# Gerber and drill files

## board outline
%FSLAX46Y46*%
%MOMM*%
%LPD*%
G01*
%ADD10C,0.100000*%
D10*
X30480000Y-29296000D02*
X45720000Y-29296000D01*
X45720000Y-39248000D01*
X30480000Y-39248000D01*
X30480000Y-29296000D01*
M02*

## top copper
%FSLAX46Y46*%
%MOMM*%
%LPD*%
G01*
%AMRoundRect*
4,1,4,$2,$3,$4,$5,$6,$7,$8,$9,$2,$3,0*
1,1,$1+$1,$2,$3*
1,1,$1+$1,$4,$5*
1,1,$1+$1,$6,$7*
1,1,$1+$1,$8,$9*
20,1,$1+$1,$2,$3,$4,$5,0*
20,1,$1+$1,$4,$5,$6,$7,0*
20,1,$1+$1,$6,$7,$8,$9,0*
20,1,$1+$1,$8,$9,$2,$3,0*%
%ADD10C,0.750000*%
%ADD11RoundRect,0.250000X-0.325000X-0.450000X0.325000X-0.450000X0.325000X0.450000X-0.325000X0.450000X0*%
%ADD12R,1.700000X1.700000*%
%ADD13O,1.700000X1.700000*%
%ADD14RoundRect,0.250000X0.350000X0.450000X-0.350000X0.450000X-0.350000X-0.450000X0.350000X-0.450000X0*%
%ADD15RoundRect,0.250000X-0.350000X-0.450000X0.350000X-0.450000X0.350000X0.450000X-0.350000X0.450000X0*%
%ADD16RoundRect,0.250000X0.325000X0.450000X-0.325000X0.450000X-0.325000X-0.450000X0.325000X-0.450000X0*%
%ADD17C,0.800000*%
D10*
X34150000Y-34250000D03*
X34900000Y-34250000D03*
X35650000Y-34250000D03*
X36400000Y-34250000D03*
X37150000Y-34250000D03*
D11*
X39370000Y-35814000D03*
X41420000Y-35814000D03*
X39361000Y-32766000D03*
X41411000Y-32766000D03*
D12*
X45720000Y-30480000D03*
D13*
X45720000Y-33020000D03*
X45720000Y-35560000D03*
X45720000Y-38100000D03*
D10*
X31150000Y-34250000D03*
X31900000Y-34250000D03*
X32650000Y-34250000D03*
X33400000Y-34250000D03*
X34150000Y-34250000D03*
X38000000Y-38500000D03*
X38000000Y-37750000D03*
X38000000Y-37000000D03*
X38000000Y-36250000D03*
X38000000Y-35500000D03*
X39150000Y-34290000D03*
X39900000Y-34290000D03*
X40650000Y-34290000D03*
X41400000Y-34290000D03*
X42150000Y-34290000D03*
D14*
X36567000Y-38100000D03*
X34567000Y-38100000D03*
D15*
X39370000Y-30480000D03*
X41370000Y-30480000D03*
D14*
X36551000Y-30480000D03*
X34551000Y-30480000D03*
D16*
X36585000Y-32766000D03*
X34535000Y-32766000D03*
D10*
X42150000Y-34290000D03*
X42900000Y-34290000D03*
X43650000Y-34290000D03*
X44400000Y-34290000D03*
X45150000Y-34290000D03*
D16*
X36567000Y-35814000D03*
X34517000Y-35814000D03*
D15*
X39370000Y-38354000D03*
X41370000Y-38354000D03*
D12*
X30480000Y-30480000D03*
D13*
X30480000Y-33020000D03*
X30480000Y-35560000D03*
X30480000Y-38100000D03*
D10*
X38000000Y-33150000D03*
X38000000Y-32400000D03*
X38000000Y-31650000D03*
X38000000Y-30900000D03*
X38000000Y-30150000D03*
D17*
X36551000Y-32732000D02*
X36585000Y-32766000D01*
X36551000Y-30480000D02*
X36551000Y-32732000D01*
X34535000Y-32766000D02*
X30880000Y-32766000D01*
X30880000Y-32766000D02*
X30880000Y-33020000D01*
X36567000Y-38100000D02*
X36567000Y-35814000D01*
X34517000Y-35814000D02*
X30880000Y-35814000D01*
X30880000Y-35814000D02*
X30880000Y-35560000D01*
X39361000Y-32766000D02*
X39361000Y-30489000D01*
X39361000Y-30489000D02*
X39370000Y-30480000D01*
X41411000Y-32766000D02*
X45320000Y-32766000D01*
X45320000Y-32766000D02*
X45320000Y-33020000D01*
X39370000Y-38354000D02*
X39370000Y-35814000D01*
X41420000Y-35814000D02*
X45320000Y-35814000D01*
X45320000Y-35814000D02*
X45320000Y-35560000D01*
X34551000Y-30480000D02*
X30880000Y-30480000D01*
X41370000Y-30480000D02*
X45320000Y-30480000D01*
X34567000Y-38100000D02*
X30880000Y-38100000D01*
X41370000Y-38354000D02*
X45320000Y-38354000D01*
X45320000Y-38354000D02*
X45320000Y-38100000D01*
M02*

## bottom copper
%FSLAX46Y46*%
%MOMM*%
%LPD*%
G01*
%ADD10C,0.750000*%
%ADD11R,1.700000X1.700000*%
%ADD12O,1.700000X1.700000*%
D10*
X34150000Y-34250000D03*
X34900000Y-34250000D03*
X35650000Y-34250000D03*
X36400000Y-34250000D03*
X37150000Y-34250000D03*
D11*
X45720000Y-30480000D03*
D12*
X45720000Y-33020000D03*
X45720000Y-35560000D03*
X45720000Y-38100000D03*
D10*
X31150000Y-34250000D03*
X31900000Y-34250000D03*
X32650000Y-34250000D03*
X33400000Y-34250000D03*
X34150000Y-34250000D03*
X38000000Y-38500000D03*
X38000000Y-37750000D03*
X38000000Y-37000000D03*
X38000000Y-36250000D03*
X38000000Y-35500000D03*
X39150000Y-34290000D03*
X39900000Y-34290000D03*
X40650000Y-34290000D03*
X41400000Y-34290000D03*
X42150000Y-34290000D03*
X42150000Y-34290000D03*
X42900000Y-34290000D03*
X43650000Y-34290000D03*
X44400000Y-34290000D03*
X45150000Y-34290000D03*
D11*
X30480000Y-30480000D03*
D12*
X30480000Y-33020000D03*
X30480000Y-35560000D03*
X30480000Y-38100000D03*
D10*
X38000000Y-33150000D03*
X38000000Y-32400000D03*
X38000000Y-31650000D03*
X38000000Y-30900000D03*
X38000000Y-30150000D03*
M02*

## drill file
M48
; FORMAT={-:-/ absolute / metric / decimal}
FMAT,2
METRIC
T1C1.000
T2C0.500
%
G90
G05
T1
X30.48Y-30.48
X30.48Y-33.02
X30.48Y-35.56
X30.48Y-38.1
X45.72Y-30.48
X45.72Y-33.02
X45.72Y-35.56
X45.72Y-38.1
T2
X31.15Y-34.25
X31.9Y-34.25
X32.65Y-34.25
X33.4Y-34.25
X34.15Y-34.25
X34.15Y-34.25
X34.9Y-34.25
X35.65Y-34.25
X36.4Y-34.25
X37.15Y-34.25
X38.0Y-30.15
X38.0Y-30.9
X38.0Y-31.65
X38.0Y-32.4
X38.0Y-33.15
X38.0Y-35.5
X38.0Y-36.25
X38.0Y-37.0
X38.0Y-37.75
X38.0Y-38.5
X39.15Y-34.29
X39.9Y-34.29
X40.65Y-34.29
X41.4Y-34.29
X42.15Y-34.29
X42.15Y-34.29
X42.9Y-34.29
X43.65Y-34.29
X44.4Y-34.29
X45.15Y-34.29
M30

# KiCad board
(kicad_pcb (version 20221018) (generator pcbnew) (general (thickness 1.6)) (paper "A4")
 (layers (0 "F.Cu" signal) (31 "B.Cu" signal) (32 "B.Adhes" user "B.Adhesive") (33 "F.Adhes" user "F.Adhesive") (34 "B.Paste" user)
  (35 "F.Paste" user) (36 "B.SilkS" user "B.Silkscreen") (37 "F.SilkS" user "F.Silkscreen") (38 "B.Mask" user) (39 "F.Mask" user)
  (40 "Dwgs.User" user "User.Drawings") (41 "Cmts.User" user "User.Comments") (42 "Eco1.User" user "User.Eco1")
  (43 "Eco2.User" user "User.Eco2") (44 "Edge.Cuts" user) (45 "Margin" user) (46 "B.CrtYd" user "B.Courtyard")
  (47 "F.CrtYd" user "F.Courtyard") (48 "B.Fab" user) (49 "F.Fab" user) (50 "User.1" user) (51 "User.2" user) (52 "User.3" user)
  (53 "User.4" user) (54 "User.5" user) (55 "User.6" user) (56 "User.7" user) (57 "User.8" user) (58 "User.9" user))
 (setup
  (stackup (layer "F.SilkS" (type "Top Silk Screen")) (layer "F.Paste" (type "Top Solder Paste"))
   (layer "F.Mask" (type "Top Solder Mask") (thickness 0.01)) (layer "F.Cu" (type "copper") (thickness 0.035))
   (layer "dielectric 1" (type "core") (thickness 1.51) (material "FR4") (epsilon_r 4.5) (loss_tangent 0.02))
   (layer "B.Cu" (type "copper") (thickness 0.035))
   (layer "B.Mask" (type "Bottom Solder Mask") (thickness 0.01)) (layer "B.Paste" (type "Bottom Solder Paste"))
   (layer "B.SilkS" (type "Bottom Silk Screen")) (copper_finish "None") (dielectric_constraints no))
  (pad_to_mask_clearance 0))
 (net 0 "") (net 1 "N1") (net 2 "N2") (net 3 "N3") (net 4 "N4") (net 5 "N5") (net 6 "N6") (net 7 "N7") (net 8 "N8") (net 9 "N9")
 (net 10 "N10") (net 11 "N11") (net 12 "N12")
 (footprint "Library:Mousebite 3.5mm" (layer "F.Cu") (at 34.15 34.25 90)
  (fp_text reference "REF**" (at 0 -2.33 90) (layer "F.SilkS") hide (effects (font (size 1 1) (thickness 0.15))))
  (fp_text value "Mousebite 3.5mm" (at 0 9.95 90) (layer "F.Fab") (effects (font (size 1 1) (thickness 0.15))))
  (pad "" np_thru_hole circle (at 0 0 90) (size 0.75 0.75) (drill 0.5) (layers "*.Cu" "*.Mask"))
  (pad "" np_thru_hole circle (at 0 0.75 90) (size 0.75 0.75) (drill 0.5) (layers "*.Cu" "*.Mask"))
  (pad "" np_thru_hole circle (at 0 1.5 90) (size 0.75 0.75) (drill 0.5) (layers "*.Cu" "*.Mask"))
  (pad "" np_thru_hole circle (at 0 2.25 90) (size 0.75 0.75) (drill 0.5) (layers "*.Cu" "*.Mask"))
  (pad "" np_thru_hole circle (at 0 3 90) (size 0.75 0.75) (drill 0.5) (layers "*.Cu" "*.Mask")))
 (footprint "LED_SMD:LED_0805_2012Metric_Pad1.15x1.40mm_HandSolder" (layer "F.Cu") (at 40.395 35.814)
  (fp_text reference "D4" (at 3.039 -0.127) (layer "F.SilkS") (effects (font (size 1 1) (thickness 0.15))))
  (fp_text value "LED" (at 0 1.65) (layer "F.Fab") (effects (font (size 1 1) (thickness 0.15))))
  (pad "1" smd roundrect (at -1.025 0) (size 1.15 1.4) (layers "F.Cu" "F.Paste" "F.Mask") (roundrect_rratio 0.217391) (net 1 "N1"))
  (pad "2" smd roundrect (at 1.025 0) (size 1.15 1.4) (layers "F.Cu" "F.Paste" "F.Mask") (roundrect_rratio 0.217391) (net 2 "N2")))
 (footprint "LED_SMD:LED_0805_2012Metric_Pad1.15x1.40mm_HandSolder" (layer "F.Cu") (at 40.386 32.766)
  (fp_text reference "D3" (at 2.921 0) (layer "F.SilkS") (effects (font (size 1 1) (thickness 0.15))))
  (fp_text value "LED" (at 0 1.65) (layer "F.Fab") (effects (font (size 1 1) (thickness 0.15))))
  (pad "1" smd roundrect (at -1.025 0) (size 1.15 1.4) (layers "F.Cu" "F.Paste" "F.Mask") (roundrect_rratio 0.217391) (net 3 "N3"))
  (pad "2" smd roundrect (at 1.025 0) (size 1.15 1.4) (layers "F.Cu" "F.Paste" "F.Mask") (roundrect_rratio 0.217391) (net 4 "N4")))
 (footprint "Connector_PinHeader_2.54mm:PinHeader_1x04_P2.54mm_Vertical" (layer "F.Cu") (at 45.72 30.48)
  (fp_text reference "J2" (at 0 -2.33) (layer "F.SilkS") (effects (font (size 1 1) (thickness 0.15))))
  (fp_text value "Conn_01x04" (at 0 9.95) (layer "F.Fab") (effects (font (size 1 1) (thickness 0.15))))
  (pad "1" thru_hole rect (at 0 0) (size 1.7 1.7) (drill 1) (layers "*.Cu" "*.Mask") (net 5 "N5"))
  (pad "2" thru_hole oval (at 0 2.54) (size 1.7 1.7) (drill 1) (layers "*.Cu" "*.Mask") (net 4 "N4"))
  (pad "3" thru_hole oval (at 0 5.08) (size 1.7 1.7) (drill 1) (layers "*.Cu" "*.Mask") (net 2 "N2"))
  (pad "4" thru_hole oval (at 0 7.62) (size 1.7 1.7) (drill 1) (layers "*.Cu" "*.Mask") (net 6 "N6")))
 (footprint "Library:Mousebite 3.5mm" (layer "F.Cu") (at 31.15 34.25 90)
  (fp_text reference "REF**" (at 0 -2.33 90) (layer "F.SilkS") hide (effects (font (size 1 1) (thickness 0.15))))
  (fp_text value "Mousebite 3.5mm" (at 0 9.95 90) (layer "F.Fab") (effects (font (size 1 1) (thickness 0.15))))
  (pad "" np_thru_hole circle (at 0 0 90) (size 0.75 0.75) (drill 0.5) (layers "*.Cu" "*.Mask"))
  (pad "" np_thru_hole circle (at 0 0.75 90) (size 0.75 0.75) (drill 0.5) (layers "*.Cu" "*.Mask"))
  (pad "" np_thru_hole circle (at 0 1.5 90) (size 0.75 0.75) (drill 0.5) (layers "*.Cu" "*.Mask"))
  (pad "" np_thru_hole circle (at 0 2.25 90) (size 0.75 0.75) (drill 0.5) (layers "*.Cu" "*.Mask"))
  (pad "" np_thru_hole circle (at 0 3 90) (size 0.75 0.75) (drill 0.5) (layers "*.Cu" "*.Mask")))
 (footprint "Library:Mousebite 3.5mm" (layer "F.Cu") (at 38 38.5 180)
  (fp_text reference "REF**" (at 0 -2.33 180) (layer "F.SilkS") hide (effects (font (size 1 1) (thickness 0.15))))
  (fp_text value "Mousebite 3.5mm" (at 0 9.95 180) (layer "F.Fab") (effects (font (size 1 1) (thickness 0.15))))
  (pad "" np_thru_hole circle (at 0 0 180) (size 0.75 0.75) (drill 0.5) (layers "*.Cu" "*.Mask"))
  (pad "" np_thru_hole circle (at 0 0.75 180) (size 0.75 0.75) (drill 0.5) (layers "*.Cu" "*.Mask"))
  (pad "" np_thru_hole circle (at 0 1.5 180) (size 0.75 0.75) (drill 0.5) (layers "*.Cu" "*.Mask"))
  (pad "" np_thru_hole circle (at 0 2.25 180) (size 0.75 0.75) (drill 0.5) (layers "*.Cu" "*.Mask"))
  (pad "" np_thru_hole circle (at 0 3 180) (size 0.75 0.75) (drill 0.5) (layers "*.Cu" "*.Mask")))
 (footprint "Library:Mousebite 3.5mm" (layer "F.Cu") (at 39.15 34.29 90)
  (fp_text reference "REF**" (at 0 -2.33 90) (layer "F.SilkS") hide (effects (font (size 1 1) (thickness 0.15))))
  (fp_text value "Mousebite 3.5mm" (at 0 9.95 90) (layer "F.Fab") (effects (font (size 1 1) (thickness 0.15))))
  (pad "" np_thru_hole circle (at 0 0 90) (size 0.75 0.75) (drill 0.5) (layers "*.Cu" "*.Mask"))
  (pad "" np_thru_hole circle (at 0 0.75 90) (size 0.75 0.75) (drill 0.5) (layers "*.Cu" "*.Mask"))
  (pad "" np_thru_hole circle (at 0 1.5 90) (size 0.75 0.75) (drill 0.5) (layers "*.Cu" "*.Mask"))
  (pad "" np_thru_hole circle (at 0 2.25 90) (size 0.75 0.75) (drill 0.5) (layers "*.Cu" "*.Mask"))
  (pad "" np_thru_hole circle (at 0 3 90) (size 0.75 0.75) (drill 0.5) (layers "*.Cu" "*.Mask")))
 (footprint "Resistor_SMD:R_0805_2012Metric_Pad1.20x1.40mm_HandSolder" (layer "F.Cu") (at 35.567 38.1 180)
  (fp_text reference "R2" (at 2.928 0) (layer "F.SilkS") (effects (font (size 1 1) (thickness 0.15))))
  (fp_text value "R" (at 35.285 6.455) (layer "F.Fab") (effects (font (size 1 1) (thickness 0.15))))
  (pad "1" smd roundrect (at -1 0 180) (size 1.2 1.4) (layers "F.Cu" "F.Paste" "F.Mask") (roundrect_rratio 0.208333) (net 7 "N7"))
  (pad "2" smd roundrect (at 1 0 180) (size 1.2 1.4) (layers "F.Cu" "F.Paste" "F.Mask") (roundrect_rratio 0.208333) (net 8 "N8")))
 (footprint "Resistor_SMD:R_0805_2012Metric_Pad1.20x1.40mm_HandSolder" (layer "F.Cu") (at 40.37 30.48)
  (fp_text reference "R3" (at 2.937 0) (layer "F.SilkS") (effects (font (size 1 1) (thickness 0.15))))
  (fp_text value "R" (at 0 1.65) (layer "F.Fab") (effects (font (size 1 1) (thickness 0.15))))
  (pad "1" smd roundrect (at -1 0) (size 1.2 1.4) (layers "F.Cu" "F.Paste" "F.Mask") (roundrect_rratio 0.208333) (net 3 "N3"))
  (pad "2" smd roundrect (at 1 0) (size 1.2 1.4) (layers "F.Cu" "F.Paste" "F.Mask") (roundrect_rratio 0.208333) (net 5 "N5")))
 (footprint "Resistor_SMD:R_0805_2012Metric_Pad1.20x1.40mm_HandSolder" (layer "F.Cu") (at 35.551 30.48 180)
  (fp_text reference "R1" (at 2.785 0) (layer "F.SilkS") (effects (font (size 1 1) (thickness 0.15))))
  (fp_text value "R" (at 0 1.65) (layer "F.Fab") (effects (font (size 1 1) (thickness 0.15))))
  (pad "1" smd roundrect (at -1 0 180) (size 1.2 1.4) (layers "F.Cu" "F.Paste" "F.Mask") (roundrect_rratio 0.208333) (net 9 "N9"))
  (pad "2" smd roundrect (at 1 0 180) (size 1.2 1.4) (layers "F.Cu" "F.Paste" "F.Mask") (roundrect_rratio 0.208333) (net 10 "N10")))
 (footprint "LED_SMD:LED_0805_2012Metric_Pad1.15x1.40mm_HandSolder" (layer "F.Cu") (at 35.56 32.766 180)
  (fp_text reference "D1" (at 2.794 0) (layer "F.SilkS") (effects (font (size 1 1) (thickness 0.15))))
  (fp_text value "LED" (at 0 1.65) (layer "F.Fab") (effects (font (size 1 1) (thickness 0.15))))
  (pad "1" smd roundrect (at -1.025 0 180) (size 1.15 1.4) (layers "F.Cu" "F.Paste" "F.Mask") (roundrect_rratio 0.217391) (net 9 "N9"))
  (pad "2" smd roundrect (at 1.025 0 180) (size 1.15 1.4) (layers "F.Cu" "F.Paste" "F.Mask") (roundrect_rratio 0.217391) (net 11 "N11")))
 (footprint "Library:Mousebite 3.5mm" (layer "F.Cu") (at 42.15 34.29 90)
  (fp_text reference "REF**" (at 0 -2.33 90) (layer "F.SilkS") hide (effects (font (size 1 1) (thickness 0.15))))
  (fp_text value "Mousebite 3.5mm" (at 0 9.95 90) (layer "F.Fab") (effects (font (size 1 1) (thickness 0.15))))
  (pad "" np_thru_hole circle (at 0 0 90) (size 0.75 0.75) (drill 0.5) (layers "*.Cu" "*.Mask"))
  (pad "" np_thru_hole circle (at 0 0.75 90) (size 0.75 0.75) (drill 0.5) (layers "*.Cu" "*.Mask"))
  (pad "" np_thru_hole circle (at 0 1.5 90) (size 0.75 0.75) (drill 0.5) (layers "*.Cu" "*.Mask"))
  (pad "" np_thru_hole circle (at 0 2.25 90) (size 0.75 0.75) (drill 0.5) (layers "*.Cu" "*.Mask"))
  (pad "" np_thru_hole circle (at 0 3 90) (size 0.75 0.75) (drill 0.5) (layers "*.Cu" "*.Mask")))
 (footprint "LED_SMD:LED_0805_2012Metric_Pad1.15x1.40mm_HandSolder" (layer "F.Cu") (at 35.542 35.814 180)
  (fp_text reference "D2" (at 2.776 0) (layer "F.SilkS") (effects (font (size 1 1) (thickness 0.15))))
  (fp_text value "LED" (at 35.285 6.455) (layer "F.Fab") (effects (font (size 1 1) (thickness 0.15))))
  (pad "1" smd roundrect (at -1.025 0 180) (size 1.15 1.4) (layers "F.Cu" "F.Paste" "F.Mask") (roundrect_rratio 0.217391) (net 7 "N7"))
  (pad "2" smd roundrect (at 1.025 0 180) (size 1.15 1.4) (layers "F.Cu" "F.Paste" "F.Mask") (roundrect_rratio 0.217391) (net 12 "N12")))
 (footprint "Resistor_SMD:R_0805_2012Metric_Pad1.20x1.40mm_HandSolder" (layer "F.Cu") (at 40.37 38.354)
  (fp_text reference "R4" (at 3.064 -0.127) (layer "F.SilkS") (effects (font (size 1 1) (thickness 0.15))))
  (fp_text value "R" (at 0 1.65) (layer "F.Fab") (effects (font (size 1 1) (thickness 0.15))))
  (pad "1" smd roundrect (at -1 0) (size 1.2 1.4) (layers "F.Cu" "F.Paste" "F.Mask") (roundrect_rratio 0.208333) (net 1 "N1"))
  (pad "2" smd roundrect (at 1 0) (size 1.2 1.4) (layers "F.Cu" "F.Paste" "F.Mask") (roundrect_rratio 0.208333) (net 6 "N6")))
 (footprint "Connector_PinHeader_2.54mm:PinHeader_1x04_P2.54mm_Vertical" (layer "F.Cu") (at 30.48 30.48)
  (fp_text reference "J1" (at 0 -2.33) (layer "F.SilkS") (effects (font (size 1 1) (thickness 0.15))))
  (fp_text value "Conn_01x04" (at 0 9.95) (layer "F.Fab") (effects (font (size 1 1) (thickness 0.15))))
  (pad "1" thru_hole rect (at 0 0) (size 1.7 1.7) (drill 1) (layers "*.Cu" "*.Mask") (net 10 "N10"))
  (pad "2" thru_hole oval (at 0 2.54) (size 1.7 1.7) (drill 1) (layers "*.Cu" "*.Mask") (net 11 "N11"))
  (pad "3" thru_hole oval (at 0 5.08) (size 1.7 1.7) (drill 1) (layers "*.Cu" "*.Mask") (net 12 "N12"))
  (pad "4" thru_hole oval (at 0 7.62) (size 1.7 1.7) (drill 1) (layers "*.Cu" "*.Mask") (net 8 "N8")))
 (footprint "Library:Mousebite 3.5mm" (layer "F.Cu") (at 38 33.15 180)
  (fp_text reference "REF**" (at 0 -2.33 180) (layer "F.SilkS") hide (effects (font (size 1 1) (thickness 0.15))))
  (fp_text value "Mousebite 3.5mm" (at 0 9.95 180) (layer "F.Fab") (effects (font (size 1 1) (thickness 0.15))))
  (pad "" np_thru_hole circle (at 0 0 180) (size 0.75 0.75) (drill 0.5) (layers "*.Cu" "*.Mask"))
  (pad "" np_thru_hole circle (at 0 0.75 180) (size 0.75 0.75) (drill 0.5) (layers "*.Cu" "*.Mask"))
  (pad "" np_thru_hole circle (at 0 1.5 180) (size 0.75 0.75) (drill 0.5) (layers "*.Cu" "*.Mask"))
  (pad "" np_thru_hole circle (at 0 2.25 180) (size 0.75 0.75) (drill 0.5) (layers "*.Cu" "*.Mask"))
  (pad "" np_thru_hole circle (at 0 3 180) (size 0.75 0.75) (drill 0.5) (layers "*.Cu" "*.Mask")))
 (gr_rect (start 30.48 29.296) (end 45.72 39.248) (stroke (width 0.1) (type default)) (fill none) (layer "Edge.Cuts"))
 (segment (start 36.551 32.732) (end 36.585 32.766) (width 0.8) (layer "F.Cu") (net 9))
 (segment (start 36.551 30.48) (end 36.551 32.732) (width 0.8) (layer "F.Cu") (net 9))
 (segment (start 34.535 32.766) (end 30.88 32.766) (width 0.8) (layer "F.Cu") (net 11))
 (segment (start 30.88 32.766) (end 30.88 33.02) (width 0.8) (layer "F.Cu") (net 11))
 (segment (start 36.567 38.1) (end 36.567 35.814) (width 0.8) (layer "F.Cu") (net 7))
 (segment (start 34.517 35.814) (end 30.88 35.814) (width 0.8) (layer "F.Cu") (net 12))
 (segment (start 30.88 35.814) (end 30.88 35.56) (width 0.8) (layer "F.Cu") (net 12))
 (segment (start 39.361 32.766) (end 39.361 30.489) (width 0.8) (layer "F.Cu") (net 3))
 (segment (start 39.361 30.489) (end 39.37 30.48) (width 0.8) (layer "F.Cu") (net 3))
 (segment (start 41.411 32.766) (end 45.32 32.766) (width 0.8) (layer "F.Cu") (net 4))
 (segment (start 45.32 32.766) (end 45.32 33.02) (width 0.8) (layer "F.Cu") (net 4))
 (segment (start 39.37 38.354) (end 39.37 35.814) (width 0.8) (layer "F.Cu") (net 1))
 (segment (start 41.42 35.814) (end 45.32 35.814) (width 0.8) (layer "F.Cu") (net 2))
 (segment (start 45.32 35.814) (end 45.32 35.56) (width 0.8) (layer "F.Cu") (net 2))
 (segment (start 34.551 30.48) (end 30.88 30.48) (width 0.8) (layer "F.Cu") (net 10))
 (segment (start 41.37 30.48) (end 45.32 30.48) (width 0.8) (layer "F.Cu") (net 5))
 (segment (start 34.567 38.1) (end 30.88 38.1) (width 0.8) (layer "F.Cu") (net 8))
 (segment (start 41.37 38.354) (end 45.32 38.354) (width 0.8) (layer "F.Cu") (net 6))
 (segment (start 45.32 38.354) (end 45.32 38.1) (width 0.8) (layer "F.Cu") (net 6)))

